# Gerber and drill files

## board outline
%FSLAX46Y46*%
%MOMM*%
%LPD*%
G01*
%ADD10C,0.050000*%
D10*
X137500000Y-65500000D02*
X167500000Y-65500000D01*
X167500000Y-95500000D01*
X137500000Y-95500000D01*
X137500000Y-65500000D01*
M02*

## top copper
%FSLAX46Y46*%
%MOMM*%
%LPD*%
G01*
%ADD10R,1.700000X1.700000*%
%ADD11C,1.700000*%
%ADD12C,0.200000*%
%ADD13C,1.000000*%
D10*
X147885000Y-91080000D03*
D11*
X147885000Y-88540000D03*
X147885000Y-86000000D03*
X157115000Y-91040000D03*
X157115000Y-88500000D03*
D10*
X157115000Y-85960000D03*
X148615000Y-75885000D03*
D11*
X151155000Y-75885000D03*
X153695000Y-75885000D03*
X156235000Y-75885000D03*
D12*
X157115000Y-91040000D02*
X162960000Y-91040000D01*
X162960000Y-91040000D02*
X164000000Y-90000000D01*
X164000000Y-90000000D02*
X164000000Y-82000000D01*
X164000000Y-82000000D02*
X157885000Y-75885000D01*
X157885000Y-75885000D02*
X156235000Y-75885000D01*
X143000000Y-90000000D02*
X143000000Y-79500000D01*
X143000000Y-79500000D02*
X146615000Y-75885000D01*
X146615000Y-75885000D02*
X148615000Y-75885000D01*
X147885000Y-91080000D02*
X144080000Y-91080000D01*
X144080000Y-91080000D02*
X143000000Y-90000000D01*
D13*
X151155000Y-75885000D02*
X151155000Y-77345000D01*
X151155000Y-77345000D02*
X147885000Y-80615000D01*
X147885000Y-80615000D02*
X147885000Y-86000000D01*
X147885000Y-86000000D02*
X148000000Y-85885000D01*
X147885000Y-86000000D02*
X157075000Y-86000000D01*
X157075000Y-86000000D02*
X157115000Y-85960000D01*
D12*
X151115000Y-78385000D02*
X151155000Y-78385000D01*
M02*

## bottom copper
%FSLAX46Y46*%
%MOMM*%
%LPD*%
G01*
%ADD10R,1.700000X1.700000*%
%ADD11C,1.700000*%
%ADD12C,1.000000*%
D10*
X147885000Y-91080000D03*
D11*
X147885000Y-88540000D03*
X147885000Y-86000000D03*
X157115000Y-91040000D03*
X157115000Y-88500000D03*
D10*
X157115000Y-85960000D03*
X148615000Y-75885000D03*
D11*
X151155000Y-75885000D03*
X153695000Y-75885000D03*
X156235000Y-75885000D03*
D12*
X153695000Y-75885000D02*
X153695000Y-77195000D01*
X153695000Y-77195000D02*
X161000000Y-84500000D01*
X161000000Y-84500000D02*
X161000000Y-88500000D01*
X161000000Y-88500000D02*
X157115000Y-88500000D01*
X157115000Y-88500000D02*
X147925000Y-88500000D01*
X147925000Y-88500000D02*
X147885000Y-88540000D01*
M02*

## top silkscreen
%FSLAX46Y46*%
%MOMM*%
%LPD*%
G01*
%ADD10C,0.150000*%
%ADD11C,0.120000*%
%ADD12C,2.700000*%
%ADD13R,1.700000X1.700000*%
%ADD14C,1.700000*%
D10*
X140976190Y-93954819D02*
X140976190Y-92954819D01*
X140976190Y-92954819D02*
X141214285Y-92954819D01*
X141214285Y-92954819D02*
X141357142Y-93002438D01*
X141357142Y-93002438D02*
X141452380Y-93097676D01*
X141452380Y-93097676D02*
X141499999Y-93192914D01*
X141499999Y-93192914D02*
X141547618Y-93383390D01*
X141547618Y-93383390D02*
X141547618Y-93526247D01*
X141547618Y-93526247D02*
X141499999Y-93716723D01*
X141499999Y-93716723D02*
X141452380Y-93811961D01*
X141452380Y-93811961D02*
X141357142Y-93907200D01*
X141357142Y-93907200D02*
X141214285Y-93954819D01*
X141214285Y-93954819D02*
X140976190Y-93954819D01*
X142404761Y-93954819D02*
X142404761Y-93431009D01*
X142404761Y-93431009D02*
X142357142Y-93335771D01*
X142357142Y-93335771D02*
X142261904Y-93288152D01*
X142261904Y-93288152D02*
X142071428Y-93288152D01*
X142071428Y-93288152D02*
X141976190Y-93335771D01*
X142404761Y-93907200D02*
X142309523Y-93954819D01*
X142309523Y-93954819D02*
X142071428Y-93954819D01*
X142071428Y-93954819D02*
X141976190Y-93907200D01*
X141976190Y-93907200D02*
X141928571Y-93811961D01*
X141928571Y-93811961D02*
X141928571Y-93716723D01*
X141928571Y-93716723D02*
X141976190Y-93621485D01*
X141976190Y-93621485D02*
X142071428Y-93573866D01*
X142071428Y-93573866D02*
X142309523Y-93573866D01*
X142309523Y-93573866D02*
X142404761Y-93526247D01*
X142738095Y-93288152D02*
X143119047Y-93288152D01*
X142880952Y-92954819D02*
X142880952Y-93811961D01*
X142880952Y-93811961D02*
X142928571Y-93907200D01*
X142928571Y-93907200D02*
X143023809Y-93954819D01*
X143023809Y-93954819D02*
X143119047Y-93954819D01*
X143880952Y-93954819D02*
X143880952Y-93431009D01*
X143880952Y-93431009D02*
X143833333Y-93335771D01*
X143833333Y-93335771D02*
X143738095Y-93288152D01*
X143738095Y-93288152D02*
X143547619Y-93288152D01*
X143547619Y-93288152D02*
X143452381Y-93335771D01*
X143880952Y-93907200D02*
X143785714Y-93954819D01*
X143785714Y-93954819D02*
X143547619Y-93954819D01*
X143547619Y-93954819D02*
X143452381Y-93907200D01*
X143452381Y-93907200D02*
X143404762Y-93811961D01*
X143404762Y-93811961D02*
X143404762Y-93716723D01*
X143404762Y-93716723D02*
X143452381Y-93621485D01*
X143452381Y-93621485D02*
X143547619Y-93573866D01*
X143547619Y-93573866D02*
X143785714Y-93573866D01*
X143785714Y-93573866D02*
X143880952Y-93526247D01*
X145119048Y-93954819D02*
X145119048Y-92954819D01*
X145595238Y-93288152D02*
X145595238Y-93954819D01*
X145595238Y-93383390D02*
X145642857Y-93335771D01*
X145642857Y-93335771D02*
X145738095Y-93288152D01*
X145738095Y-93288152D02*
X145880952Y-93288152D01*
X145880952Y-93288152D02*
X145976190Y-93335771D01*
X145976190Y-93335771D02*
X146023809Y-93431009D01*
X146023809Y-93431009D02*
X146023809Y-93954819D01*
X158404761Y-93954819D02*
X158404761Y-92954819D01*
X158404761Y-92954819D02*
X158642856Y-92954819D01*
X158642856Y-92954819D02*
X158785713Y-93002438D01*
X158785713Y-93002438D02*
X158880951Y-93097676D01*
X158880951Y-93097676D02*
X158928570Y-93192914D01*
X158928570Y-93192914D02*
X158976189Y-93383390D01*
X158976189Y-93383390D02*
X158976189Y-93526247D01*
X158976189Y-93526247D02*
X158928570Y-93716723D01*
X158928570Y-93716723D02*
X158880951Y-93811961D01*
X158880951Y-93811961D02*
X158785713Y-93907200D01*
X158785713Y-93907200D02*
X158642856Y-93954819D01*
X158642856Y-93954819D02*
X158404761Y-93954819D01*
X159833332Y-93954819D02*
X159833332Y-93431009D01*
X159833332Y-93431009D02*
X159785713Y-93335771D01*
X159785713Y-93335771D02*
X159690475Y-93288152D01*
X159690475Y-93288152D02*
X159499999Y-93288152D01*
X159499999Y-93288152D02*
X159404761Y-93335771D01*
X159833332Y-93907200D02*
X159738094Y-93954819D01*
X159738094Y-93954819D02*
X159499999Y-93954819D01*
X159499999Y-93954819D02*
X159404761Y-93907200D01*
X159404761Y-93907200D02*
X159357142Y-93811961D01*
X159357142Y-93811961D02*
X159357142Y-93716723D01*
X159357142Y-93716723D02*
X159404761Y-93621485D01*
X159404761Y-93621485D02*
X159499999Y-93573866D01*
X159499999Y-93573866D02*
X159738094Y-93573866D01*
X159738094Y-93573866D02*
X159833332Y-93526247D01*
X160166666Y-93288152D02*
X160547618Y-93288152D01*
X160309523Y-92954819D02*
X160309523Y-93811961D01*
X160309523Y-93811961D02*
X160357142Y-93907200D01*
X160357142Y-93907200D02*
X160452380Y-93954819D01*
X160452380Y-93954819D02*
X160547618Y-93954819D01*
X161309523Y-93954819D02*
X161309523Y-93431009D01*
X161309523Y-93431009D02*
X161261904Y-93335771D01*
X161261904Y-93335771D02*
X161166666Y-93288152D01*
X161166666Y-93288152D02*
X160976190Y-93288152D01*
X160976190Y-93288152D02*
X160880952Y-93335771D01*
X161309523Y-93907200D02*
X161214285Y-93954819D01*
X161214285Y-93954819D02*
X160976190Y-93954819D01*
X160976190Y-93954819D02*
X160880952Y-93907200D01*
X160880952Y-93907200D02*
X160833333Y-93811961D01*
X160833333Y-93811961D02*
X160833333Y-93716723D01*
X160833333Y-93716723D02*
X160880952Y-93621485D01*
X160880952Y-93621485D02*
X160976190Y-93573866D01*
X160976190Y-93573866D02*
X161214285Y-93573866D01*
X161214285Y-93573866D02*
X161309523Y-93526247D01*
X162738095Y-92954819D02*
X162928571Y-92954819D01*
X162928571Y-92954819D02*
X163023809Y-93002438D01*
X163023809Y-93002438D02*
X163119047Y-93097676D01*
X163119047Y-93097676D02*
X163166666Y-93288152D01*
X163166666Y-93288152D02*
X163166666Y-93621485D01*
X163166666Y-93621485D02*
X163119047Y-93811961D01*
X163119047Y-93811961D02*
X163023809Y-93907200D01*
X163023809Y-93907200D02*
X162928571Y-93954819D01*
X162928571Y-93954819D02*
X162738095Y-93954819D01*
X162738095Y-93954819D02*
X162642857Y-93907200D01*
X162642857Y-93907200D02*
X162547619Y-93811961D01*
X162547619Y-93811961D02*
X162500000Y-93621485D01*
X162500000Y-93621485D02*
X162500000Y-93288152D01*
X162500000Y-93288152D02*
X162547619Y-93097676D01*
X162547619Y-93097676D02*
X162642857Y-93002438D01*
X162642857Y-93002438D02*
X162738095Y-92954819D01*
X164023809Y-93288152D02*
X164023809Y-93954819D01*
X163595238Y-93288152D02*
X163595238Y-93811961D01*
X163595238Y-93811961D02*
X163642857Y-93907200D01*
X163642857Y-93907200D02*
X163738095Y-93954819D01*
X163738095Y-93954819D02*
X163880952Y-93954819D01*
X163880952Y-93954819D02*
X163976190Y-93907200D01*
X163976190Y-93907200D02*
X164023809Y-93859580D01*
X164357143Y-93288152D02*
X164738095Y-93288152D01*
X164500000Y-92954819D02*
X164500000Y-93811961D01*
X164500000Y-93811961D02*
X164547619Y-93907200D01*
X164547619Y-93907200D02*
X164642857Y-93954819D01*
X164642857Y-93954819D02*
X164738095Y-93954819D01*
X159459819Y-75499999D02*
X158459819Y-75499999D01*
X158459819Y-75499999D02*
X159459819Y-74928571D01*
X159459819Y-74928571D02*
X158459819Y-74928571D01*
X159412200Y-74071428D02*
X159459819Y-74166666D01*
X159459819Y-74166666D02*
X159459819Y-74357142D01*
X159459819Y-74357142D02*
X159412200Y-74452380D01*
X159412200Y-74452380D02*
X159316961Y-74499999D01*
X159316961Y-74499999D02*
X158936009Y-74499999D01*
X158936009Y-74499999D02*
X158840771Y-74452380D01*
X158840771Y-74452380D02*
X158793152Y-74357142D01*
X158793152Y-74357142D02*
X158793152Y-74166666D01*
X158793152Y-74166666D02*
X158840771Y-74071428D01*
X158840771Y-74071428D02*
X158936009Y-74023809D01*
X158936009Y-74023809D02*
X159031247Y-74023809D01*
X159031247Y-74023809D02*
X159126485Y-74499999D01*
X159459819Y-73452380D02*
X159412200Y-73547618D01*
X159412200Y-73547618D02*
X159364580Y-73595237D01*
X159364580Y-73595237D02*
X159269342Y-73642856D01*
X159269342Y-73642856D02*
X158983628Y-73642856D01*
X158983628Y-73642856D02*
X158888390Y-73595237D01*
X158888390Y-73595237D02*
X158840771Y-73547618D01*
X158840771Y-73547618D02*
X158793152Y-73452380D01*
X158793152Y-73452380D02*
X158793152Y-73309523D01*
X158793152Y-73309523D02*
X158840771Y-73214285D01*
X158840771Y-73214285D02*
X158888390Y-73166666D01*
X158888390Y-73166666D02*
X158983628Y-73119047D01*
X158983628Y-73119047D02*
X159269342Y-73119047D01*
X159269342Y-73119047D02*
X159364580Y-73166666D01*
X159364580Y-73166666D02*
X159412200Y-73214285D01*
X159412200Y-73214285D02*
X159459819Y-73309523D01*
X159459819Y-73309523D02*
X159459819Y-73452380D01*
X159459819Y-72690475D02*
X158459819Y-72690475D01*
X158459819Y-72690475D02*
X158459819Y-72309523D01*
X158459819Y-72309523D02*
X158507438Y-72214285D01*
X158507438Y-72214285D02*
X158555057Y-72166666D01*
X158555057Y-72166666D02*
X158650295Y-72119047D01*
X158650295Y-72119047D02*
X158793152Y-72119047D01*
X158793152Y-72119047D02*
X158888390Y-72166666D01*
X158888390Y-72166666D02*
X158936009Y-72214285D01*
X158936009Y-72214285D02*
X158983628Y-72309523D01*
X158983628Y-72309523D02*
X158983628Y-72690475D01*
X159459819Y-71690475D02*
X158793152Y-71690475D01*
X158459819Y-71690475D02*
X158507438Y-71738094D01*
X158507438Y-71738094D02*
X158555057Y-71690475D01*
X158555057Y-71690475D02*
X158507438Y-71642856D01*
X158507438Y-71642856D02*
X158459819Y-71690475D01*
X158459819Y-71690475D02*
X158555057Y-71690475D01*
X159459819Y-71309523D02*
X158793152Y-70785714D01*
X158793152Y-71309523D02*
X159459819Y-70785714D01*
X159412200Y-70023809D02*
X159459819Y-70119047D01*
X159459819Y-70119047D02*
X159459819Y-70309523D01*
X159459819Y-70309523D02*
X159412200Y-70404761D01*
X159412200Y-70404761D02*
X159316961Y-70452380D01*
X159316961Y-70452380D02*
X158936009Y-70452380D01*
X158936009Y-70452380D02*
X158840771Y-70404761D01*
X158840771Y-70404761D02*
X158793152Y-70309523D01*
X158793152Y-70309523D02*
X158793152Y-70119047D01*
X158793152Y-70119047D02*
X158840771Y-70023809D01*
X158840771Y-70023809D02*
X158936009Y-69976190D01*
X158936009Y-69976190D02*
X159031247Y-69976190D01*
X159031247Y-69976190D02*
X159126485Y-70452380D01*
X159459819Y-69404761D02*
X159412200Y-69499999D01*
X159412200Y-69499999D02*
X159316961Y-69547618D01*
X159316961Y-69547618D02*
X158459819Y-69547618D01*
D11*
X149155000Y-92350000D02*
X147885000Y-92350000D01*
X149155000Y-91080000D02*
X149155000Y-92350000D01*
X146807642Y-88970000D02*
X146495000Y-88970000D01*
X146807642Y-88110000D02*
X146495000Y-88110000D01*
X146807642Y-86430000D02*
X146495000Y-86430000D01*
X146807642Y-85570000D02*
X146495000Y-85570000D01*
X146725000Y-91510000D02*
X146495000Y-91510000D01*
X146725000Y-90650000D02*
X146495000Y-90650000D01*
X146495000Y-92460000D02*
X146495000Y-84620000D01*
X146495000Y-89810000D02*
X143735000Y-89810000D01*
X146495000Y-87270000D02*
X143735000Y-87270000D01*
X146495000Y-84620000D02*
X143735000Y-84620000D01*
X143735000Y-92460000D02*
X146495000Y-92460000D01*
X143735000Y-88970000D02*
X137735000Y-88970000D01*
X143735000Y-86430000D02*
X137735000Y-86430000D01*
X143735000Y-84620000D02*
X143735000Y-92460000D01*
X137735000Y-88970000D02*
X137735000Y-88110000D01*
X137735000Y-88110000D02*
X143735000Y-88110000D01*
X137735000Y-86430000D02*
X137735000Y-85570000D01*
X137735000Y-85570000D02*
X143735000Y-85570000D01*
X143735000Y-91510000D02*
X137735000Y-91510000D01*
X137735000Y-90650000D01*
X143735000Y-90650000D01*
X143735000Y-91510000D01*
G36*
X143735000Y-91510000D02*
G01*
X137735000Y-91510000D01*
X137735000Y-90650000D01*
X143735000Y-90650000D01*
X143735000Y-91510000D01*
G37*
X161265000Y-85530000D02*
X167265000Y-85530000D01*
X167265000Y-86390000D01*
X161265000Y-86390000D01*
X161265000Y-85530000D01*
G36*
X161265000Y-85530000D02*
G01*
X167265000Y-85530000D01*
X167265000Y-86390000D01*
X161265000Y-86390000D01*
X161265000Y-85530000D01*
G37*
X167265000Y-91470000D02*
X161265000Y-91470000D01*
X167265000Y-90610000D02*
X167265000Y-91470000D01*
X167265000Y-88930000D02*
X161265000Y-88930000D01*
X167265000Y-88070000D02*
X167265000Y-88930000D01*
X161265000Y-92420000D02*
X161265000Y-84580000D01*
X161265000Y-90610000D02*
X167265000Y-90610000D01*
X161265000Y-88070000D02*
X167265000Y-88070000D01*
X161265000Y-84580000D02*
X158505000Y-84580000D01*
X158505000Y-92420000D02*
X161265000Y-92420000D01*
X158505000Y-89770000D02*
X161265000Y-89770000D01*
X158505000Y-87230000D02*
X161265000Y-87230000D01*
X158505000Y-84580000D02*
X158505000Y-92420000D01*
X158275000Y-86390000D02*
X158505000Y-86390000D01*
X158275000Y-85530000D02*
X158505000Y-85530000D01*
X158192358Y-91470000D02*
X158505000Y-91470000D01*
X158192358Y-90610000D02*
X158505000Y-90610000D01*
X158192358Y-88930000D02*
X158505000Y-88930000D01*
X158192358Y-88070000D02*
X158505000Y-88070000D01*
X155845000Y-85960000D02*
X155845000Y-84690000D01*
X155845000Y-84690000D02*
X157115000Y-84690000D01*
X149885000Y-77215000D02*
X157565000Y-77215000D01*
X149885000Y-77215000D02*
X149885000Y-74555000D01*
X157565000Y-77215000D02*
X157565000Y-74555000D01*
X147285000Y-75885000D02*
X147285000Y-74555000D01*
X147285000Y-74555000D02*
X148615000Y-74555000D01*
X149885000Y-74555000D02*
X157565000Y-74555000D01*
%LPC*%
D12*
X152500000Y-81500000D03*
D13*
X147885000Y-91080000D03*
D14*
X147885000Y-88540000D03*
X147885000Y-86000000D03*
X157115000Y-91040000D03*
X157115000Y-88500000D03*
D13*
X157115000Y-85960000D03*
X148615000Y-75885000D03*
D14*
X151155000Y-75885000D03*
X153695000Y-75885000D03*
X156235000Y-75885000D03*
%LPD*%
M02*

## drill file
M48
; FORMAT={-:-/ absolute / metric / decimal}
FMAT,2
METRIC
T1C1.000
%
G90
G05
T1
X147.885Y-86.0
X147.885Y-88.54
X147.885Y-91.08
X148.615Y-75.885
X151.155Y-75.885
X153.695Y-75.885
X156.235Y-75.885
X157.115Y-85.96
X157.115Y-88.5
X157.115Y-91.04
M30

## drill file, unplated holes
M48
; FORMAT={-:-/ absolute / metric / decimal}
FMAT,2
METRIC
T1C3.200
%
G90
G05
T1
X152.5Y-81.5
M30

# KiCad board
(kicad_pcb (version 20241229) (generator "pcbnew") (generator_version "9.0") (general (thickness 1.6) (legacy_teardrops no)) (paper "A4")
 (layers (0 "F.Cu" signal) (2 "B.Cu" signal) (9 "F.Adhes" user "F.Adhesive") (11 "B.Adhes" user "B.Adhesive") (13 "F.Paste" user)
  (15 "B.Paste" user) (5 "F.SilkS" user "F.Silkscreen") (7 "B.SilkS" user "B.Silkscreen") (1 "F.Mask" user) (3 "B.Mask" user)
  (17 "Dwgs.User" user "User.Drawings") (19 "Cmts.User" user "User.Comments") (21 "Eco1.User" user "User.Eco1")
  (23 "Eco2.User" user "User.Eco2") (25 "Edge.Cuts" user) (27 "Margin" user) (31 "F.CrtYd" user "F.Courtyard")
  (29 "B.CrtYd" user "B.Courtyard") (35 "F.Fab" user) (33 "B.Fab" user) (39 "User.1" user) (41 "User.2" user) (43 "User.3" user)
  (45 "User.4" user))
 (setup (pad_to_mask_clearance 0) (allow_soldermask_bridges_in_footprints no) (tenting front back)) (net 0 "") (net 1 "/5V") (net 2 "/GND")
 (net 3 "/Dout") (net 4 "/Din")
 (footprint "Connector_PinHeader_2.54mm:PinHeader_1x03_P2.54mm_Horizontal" (layer "F.Cu") (at 157.115 85.96)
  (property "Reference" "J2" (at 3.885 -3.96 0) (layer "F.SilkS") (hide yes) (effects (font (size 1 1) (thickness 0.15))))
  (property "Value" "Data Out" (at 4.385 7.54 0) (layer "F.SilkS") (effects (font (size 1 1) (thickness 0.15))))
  (fp_line (start -1.27 -1.27) (end 0 -1.27) (stroke (width 0.12) (type solid)) (layer "F.SilkS"))
  (fp_line (start -1.27 0) (end -1.27 -1.27) (stroke (width 0.12) (type solid)) (layer "F.SilkS"))
  (fp_line (start 1.077358 2.11) (end 1.39 2.11) (stroke (width 0.12) (type solid)) (layer "F.SilkS"))
  (fp_line (start 1.077358 2.97) (end 1.39 2.97) (stroke (width 0.12) (type solid)) (layer "F.SilkS"))
  (fp_line (start 1.077358 4.65) (end 1.39 4.65) (stroke (width 0.12) (type solid)) (layer "F.SilkS"))
  (fp_line (start 1.077358 5.51) (end 1.39 5.51) (stroke (width 0.12) (type solid)) (layer "F.SilkS"))
  (fp_line (start 1.16 -0.43) (end 1.39 -0.43) (stroke (width 0.12) (type solid)) (layer "F.SilkS"))
  (fp_line (start 1.16 0.43) (end 1.39 0.43) (stroke (width 0.12) (type solid)) (layer "F.SilkS"))
  (fp_line (start 1.39 -1.38) (end 1.39 6.46) (stroke (width 0.12) (type solid)) (layer "F.SilkS"))
  (fp_line (start 1.39 1.27) (end 4.15 1.27) (stroke (width 0.12) (type solid)) (layer "F.SilkS"))
  (fp_line (start 1.39 3.81) (end 4.15 3.81) (stroke (width 0.12) (type solid)) (layer "F.SilkS"))
  (fp_line (start 1.39 6.46) (end 4.15 6.46) (stroke (width 0.12) (type solid)) (layer "F.SilkS"))
  (fp_line (start 4.15 -1.38) (end 1.39 -1.38) (stroke (width 0.12) (type solid)) (layer "F.SilkS"))
  (fp_line (start 4.15 2.11) (end 10.15 2.11) (stroke (width 0.12) (type solid)) (layer "F.SilkS"))
  (fp_line (start 4.15 4.65) (end 10.15 4.65) (stroke (width 0.12) (type solid)) (layer "F.SilkS"))
  (fp_line (start 4.15 6.46) (end 4.15 -1.38) (stroke (width 0.12) (type solid)) (layer "F.SilkS"))
  (fp_line (start 10.15 2.11) (end 10.15 2.97) (stroke (width 0.12) (type solid)) (layer "F.SilkS"))
  (fp_line (start 10.15 2.97) (end 4.15 2.97) (stroke (width 0.12) (type solid)) (layer "F.SilkS"))
  (fp_line (start 10.15 4.65) (end 10.15 5.51) (stroke (width 0.12) (type solid)) (layer "F.SilkS"))
  (fp_line (start 10.15 5.51) (end 4.15 5.51) (stroke (width 0.12) (type solid)) (layer "F.SilkS"))
  (fp_rect (start 4.15 -0.43) (end 10.15 0.43) (stroke (width 0.12) (type solid)) (fill yes) (layer "F.SilkS"))
  (pad "1" thru_hole rect (at 0 0) (size 1.7 1.7) (drill 1) (layers "*.Cu" "*.Mask") (remove_unused_layers no) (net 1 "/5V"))
  (pad "2" thru_hole circle (at 0 2.54) (size 1.7 1.7) (drill 1) (layers "*.Cu" "*.Mask") (remove_unused_layers no) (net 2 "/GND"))
  (pad "3" thru_hole circle (at 0 5.08) (size 1.7 1.7) (drill 1) (layers "*.Cu" "*.Mask") (remove_unused_layers no) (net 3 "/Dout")))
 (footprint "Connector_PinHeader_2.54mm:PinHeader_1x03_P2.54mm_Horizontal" (layer "F.Cu") (at 147.885 91.08 180)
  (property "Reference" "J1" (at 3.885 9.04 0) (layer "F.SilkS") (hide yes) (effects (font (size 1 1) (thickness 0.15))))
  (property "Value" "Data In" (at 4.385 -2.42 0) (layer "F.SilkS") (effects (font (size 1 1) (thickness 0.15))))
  (fp_line (start 10.15 5.51) (end 4.15 5.51) (stroke (width 0.12) (type solid)) (layer "F.SilkS"))
  (fp_line (start 10.15 4.65) (end 10.15 5.51) (stroke (width 0.12) (type solid)) (layer "F.SilkS"))
  (fp_line (start 10.15 2.97) (end 4.15 2.97) (stroke (width 0.12) (type solid)) (layer "F.SilkS"))
  (fp_line (start 10.15 2.11) (end 10.15 2.97) (stroke (width 0.12) (type solid)) (layer "F.SilkS"))
  (fp_line (start 4.15 6.46) (end 4.15 -1.38) (stroke (width 0.12) (type solid)) (layer "F.SilkS"))
  (fp_line (start 4.15 4.65) (end 10.15 4.65) (stroke (width 0.12) (type solid)) (layer "F.SilkS"))
  (fp_line (start 4.15 2.11) (end 10.15 2.11) (stroke (width 0.12) (type solid)) (layer "F.SilkS"))
  (fp_line (start 4.15 -1.38) (end 1.39 -1.38) (stroke (width 0.12) (type solid)) (layer "F.SilkS"))
  (fp_line (start 1.39 6.46) (end 4.15 6.46) (stroke (width 0.12) (type solid)) (layer "F.SilkS"))
  (fp_line (start 1.39 3.81) (end 4.15 3.81) (stroke (width 0.12) (type solid)) (layer "F.SilkS"))
  (fp_line (start 1.39 1.27) (end 4.15 1.27) (stroke (width 0.12) (type solid)) (layer "F.SilkS"))
  (fp_line (start 1.39 -1.38) (end 1.39 6.46) (stroke (width 0.12) (type solid)) (layer "F.SilkS"))
  (fp_line (start 1.16 0.43) (end 1.39 0.43) (stroke (width 0.12) (type solid)) (layer "F.SilkS"))
  (fp_line (start 1.16 -0.43) (end 1.39 -0.43) (stroke (width 0.12) (type solid)) (layer "F.SilkS"))
  (fp_line (start 1.077358 5.51) (end 1.39 5.51) (stroke (width 0.12) (type solid)) (layer "F.SilkS"))
  (fp_line (start 1.077358 4.65) (end 1.39 4.65) (stroke (width 0.12) (type solid)) (layer "F.SilkS"))
  (fp_line (start 1.077358 2.97) (end 1.39 2.97) (stroke (width 0.12) (type solid)) (layer "F.SilkS"))
  (fp_line (start 1.077358 2.11) (end 1.39 2.11) (stroke (width 0.12) (type solid)) (layer "F.SilkS"))
  (fp_line (start -1.27 0) (end -1.27 -1.27) (stroke (width 0.12) (type solid)) (layer "F.SilkS"))
  (fp_line (start -1.27 -1.27) (end 0 -1.27) (stroke (width 0.12) (type solid)) (layer "F.SilkS"))
  (fp_rect (start 4.15 -0.43) (end 10.15 0.43) (stroke (width 0.12) (type solid)) (fill yes) (layer "F.SilkS"))
  (pad "1" thru_hole rect (at 0 0 180) (size 1.7 1.7) (drill 1) (layers "*.Cu" "*.Mask") (remove_unused_layers no) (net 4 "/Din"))
  (pad "2" thru_hole circle (at 0 2.54 180) (size 1.7 1.7) (drill 1) (layers "*.Cu" "*.Mask") (remove_unused_layers no) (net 2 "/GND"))
  (pad "3" thru_hole circle (at 0 5.08 180) (size 1.7 1.7) (drill 1) (layers "*.Cu" "*.Mask") (remove_unused_layers no) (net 1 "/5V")))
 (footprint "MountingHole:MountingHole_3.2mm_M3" (layer "F.Cu") (at 152.5 81.5)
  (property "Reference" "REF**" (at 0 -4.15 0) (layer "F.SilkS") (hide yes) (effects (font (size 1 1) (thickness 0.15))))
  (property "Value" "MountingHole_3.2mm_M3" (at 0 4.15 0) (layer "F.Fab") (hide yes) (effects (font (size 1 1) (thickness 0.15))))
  (pad "" np_thru_hole circle (at 0 0) (size 2.7 2.7) (drill 3.2) (layers "*.Cu" "*.Mask")))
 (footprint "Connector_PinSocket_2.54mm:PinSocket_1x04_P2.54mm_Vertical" (layer "F.Cu") (at 148.615 75.885 90)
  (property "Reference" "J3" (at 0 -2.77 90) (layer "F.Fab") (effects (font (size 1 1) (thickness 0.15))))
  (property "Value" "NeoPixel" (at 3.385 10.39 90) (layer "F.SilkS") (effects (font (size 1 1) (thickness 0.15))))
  (fp_line (start 1.33 -1.33) (end 1.33 0) (stroke (width 0.12) (type solid)) (layer "F.SilkS"))
  (fp_line (start 0 -1.33) (end 1.33 -1.33) (stroke (width 0.12) (type solid)) (layer "F.SilkS"))
  (fp_line (start 1.33 1.27) (end 1.33 8.95) (stroke (width 0.12) (type solid)) (layer "F.SilkS"))
  (fp_line (start -1.33 1.27) (end 1.33 1.27) (stroke (width 0.12) (type solid)) (layer "F.SilkS"))
  (fp_line (start -1.33 1.27) (end -1.33 8.95) (stroke (width 0.12) (type solid)) (layer "F.SilkS"))
  (fp_line (start -1.33 8.95) (end 1.33 8.95) (stroke (width 0.12) (type solid)) (layer "F.SilkS"))
  (pad "1" thru_hole rect (at 0 0 90) (size 1.7 1.7) (drill 1) (layers "*.Cu" "*.Mask") (remove_unused_layers no) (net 4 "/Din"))
  (pad "2" thru_hole circle (at 0 2.54 90) (size 1.7 1.7) (drill 1) (layers "*.Cu" "*.Mask") (remove_unused_layers no) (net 1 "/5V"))
  (pad "3" thru_hole circle (at 0 5.08 90) (size 1.7 1.7) (drill 1) (layers "*.Cu" "*.Mask") (remove_unused_layers no) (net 2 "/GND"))
  (pad "4" thru_hole circle (at 0 7.62 90) (size 1.7 1.7) (drill 1) (layers "*.Cu" "*.Mask") (remove_unused_layers no) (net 3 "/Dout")))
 (gr_rect (start 137.5 65.5) (end 167.5 95.5) (stroke (width 0.05) (type solid)) (fill no) (layer "Edge.Cuts"))
 (segment (start 147.885 91.08) (end 144.08 91.08) (width 0.2) (layer "F.Cu") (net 4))
 (segment (start 144.08 91.08) (end 143 90) (width 0.2) (layer "F.Cu") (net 4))
 (segment (start 143 90) (end 143 79.5) (width 0.2) (layer "F.Cu") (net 4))
 (segment (start 146.615 75.885) (end 148.615 75.885) (width 0.2) (layer "F.Cu") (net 4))
 (segment (start 143 79.5) (end 146.615 75.885) (width 0.2) (layer "F.Cu") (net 4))
 (segment (start 157.075 86) (end 157.115 85.96) (width 1) (layer "F.Cu") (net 1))
 (segment (start 147.885 86) (end 148 85.885) (width 1) (layer "F.Cu") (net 1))
 (segment (start 151.155 77.345) (end 147.885 80.615) (width 1) (layer "F.Cu") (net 1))
 (segment (start 151.155 75.885) (end 151.155 77.345) (width 1) (layer "F.Cu") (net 1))
 (segment (start 147.885 80.615) (end 147.885 86) (width 1) (layer "F.Cu") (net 1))
 (segment (start 151.115 78.385) (end 151.155 78.385) (width 0.2) (layer "F.Cu") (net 1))
 (segment (start 147.885 86) (end 157.075 86) (width 1) (layer "F.Cu") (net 1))
 (segment (start 147.925 88.5) (end 147.885 88.54) (width 1) (layer "B.Cu") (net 2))
 (segment (start 153.695 77.195) (end 161 84.5) (width 1) (layer "B.Cu") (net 2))
 (segment (start 157.115 88.5) (end 147.925 88.5) (width 1) (layer "B.Cu") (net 2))
 (segment (start 153.695 75.885) (end 153.695 77.195) (width 1) (layer "B.Cu") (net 2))
 (segment (start 161 84.5) (end 161 88.5) (width 1) (layer "B.Cu") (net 2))
 (segment (start 161 88.5) (end 157.115 88.5) (width 1) (layer "B.Cu") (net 2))
 (segment (start 157.885 75.885) (end 156.235 75.885) (width 0.2) (layer "F.Cu") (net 3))
 (segment (start 162.96 91.04) (end 164 90) (width 0.2) (layer "F.Cu") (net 3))
 (segment (start 164 82) (end 157.885 75.885) (width 0.2) (layer "F.Cu") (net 3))
 (segment (start 157.115 91.04) (end 162.96 91.04) (width 0.2) (layer "F.Cu") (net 3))
 (segment (start 164 90) (end 164 82) (width 0.2) (layer "F.Cu") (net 3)))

